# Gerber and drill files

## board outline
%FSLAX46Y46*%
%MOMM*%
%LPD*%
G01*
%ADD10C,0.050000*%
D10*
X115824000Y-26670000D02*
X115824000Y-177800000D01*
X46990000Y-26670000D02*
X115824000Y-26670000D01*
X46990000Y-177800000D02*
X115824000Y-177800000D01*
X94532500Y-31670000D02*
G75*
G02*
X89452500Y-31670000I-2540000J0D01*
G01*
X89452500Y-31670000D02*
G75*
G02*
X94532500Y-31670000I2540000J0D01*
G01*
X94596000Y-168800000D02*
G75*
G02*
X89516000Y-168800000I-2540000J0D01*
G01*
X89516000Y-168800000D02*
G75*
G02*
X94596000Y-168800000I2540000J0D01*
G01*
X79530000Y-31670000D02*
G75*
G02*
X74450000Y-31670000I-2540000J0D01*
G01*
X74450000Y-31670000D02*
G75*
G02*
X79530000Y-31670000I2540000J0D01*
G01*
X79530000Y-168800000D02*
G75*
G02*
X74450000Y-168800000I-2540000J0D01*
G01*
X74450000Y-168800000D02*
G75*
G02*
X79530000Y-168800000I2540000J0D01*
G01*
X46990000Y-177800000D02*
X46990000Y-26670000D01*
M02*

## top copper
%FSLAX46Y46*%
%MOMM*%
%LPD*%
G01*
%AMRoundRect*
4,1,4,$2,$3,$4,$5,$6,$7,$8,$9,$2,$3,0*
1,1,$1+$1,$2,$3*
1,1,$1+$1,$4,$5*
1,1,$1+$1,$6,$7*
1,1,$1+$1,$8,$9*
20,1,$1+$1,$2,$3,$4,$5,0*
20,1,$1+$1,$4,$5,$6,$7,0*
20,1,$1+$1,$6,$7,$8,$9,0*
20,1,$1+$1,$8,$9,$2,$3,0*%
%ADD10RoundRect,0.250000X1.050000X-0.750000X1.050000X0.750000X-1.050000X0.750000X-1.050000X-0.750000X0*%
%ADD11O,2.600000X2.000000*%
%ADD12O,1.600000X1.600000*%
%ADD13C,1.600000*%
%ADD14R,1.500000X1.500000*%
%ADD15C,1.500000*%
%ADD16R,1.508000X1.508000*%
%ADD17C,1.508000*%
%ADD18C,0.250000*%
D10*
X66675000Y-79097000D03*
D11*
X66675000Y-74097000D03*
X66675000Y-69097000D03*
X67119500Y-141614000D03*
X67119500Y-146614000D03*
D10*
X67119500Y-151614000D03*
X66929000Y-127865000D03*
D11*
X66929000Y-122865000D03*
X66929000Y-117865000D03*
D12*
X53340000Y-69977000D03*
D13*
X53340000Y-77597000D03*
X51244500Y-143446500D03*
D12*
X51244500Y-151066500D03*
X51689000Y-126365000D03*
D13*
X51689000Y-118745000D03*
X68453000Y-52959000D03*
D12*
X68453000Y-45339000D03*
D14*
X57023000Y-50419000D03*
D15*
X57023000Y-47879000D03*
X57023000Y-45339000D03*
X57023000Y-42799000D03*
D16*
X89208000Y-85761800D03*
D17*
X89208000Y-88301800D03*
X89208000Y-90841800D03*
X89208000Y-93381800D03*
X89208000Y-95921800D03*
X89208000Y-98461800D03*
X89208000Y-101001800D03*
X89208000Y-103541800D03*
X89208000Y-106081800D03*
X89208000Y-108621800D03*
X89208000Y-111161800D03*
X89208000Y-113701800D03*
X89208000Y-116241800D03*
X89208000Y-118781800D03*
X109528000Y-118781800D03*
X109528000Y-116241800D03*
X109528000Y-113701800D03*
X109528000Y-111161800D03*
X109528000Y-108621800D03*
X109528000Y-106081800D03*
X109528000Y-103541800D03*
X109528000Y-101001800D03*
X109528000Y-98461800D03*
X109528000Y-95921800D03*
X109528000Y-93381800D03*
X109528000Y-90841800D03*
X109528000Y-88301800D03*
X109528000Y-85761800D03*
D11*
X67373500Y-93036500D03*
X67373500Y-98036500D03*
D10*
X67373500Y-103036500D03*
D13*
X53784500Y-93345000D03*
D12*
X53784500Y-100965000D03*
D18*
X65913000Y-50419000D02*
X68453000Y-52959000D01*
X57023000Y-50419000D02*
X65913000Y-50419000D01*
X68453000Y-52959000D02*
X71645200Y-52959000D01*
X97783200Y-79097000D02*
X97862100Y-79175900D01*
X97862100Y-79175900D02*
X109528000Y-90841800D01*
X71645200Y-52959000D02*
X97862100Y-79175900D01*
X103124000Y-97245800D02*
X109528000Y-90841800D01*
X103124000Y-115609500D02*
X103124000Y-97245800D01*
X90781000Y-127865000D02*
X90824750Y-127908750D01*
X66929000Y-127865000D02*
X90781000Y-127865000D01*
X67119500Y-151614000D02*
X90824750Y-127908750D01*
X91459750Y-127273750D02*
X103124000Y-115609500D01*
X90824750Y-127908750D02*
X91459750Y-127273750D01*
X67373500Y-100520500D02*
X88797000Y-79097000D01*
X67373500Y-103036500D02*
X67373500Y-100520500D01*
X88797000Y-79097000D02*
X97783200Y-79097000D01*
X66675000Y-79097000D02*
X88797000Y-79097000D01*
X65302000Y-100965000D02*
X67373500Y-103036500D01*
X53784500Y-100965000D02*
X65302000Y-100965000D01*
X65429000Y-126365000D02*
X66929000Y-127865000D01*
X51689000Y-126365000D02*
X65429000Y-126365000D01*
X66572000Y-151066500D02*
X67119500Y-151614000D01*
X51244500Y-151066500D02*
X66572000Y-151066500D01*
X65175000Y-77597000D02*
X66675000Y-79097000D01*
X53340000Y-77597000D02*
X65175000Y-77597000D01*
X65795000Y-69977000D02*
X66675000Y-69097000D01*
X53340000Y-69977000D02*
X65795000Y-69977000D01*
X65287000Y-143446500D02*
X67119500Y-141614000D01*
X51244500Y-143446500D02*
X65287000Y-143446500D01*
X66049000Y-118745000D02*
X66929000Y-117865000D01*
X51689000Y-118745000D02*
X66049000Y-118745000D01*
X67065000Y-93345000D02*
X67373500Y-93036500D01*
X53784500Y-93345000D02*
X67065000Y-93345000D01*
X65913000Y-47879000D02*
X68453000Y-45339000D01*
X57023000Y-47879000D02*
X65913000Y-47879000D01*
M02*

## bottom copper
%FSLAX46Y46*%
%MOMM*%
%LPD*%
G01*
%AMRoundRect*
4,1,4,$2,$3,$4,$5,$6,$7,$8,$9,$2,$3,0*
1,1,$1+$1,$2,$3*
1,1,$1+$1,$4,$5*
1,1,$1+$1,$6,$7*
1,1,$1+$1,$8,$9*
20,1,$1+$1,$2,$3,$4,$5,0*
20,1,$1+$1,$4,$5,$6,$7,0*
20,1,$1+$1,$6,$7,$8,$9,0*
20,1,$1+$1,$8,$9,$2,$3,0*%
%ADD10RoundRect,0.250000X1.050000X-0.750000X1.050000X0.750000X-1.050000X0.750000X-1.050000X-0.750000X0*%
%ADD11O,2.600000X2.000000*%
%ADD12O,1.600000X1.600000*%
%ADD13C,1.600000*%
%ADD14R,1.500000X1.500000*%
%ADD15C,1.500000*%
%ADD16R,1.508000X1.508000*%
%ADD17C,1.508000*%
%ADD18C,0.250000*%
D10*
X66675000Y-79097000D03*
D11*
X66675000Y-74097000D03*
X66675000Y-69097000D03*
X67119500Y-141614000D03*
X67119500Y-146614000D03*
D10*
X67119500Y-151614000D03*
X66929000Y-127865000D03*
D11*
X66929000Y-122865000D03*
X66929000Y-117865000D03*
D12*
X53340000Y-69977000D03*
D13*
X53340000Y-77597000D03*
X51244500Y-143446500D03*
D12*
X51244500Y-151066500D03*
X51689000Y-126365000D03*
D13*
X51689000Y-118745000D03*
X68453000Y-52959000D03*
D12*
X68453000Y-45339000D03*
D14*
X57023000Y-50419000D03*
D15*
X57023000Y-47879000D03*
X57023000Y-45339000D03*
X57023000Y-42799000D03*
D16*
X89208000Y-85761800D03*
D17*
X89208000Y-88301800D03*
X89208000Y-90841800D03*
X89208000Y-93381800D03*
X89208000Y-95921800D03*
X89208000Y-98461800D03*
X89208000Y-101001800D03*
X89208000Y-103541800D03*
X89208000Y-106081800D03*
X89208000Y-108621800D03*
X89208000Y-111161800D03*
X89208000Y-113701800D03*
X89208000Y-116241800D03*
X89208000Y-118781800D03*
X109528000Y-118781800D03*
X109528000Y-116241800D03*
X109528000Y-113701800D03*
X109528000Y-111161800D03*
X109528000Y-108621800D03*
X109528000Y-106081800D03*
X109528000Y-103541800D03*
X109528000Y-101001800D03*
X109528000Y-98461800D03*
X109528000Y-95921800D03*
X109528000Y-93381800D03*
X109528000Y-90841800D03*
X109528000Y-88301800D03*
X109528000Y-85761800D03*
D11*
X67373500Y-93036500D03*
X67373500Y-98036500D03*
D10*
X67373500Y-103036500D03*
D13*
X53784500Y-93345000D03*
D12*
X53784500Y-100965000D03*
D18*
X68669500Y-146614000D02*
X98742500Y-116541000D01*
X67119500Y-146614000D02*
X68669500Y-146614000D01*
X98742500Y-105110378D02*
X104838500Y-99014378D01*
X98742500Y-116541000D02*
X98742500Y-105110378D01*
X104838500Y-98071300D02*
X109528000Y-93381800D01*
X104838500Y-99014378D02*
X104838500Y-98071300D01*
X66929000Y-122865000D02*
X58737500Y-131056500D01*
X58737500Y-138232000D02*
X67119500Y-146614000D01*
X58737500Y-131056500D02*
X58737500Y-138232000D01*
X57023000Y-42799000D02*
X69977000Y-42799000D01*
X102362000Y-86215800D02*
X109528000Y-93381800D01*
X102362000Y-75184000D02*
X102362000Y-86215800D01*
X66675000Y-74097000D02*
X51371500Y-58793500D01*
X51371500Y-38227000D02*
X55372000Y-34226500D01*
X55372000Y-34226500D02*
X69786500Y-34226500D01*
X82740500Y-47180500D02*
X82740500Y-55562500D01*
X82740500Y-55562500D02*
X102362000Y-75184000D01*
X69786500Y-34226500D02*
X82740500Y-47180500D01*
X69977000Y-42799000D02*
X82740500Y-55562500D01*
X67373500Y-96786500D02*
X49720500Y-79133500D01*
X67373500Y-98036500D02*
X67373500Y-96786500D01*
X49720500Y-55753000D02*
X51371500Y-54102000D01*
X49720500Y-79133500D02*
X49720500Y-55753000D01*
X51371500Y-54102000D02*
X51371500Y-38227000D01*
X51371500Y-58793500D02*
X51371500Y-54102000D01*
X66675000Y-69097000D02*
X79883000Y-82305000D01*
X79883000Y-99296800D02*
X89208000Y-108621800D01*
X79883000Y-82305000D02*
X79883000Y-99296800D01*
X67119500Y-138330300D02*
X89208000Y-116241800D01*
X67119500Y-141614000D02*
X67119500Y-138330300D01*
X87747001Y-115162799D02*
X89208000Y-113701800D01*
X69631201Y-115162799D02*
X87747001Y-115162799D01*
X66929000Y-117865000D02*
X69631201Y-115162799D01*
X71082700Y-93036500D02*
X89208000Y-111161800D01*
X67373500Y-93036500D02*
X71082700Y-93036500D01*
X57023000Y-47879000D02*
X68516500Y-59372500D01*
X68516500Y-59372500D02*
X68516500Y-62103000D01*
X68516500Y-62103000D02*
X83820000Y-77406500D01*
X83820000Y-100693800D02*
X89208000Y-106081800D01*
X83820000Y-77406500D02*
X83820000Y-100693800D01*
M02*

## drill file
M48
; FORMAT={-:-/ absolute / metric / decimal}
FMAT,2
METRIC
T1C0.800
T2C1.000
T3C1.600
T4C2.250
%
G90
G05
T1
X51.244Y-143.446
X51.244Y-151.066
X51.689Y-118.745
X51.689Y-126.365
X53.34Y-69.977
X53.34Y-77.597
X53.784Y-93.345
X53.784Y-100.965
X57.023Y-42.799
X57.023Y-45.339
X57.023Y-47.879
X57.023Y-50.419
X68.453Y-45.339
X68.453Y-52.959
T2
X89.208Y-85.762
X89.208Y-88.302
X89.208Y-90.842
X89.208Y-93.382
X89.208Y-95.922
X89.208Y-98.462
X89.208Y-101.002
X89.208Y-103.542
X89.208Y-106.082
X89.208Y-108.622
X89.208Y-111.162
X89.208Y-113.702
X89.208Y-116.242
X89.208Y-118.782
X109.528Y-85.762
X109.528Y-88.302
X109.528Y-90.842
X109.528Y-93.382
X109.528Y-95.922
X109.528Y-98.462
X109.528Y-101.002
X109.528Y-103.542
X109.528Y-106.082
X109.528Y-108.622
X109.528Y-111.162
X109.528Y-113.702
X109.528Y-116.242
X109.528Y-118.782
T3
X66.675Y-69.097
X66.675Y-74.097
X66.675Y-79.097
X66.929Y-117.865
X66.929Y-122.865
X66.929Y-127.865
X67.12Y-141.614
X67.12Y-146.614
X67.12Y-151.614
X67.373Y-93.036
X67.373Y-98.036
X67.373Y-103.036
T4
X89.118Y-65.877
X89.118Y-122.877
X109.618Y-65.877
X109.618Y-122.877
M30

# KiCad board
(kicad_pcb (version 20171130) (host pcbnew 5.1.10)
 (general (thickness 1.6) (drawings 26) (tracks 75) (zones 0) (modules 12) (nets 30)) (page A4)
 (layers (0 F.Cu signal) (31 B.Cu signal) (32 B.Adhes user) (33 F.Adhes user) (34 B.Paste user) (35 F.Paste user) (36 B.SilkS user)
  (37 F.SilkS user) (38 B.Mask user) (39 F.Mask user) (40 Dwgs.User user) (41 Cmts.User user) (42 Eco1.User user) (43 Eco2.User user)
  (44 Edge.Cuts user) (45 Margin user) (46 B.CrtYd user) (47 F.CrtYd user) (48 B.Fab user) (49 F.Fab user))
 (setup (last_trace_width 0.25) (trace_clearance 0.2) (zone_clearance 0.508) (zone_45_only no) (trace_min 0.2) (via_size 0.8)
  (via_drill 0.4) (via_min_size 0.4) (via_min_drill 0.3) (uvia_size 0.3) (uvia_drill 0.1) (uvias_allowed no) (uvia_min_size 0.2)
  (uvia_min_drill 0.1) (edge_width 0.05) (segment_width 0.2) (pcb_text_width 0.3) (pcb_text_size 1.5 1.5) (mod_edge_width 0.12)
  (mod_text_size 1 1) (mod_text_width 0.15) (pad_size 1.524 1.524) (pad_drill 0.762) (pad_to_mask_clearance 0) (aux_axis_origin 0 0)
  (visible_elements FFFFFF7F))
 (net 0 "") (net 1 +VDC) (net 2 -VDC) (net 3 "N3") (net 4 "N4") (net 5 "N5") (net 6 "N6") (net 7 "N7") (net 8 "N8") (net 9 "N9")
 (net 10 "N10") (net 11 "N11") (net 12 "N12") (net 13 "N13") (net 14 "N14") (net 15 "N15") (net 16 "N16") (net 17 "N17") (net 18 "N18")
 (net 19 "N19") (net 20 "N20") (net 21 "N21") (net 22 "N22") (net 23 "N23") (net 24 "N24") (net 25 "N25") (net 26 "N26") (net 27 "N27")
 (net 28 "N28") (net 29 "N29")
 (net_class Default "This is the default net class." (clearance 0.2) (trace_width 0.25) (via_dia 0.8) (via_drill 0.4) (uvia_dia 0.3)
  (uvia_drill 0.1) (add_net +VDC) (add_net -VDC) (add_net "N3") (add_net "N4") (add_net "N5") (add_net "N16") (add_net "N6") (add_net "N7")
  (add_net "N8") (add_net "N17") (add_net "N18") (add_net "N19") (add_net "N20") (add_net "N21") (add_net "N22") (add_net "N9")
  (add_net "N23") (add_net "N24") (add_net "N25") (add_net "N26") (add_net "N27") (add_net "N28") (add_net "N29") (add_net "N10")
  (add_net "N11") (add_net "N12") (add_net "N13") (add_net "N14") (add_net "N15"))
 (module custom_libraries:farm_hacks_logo (layer F.Cu) (at 102.108 146.304)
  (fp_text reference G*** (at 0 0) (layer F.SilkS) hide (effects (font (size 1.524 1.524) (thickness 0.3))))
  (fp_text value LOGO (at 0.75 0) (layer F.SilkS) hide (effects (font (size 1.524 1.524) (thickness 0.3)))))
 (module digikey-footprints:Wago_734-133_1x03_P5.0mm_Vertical (layer F.Cu) (at 66.675 77.597 90)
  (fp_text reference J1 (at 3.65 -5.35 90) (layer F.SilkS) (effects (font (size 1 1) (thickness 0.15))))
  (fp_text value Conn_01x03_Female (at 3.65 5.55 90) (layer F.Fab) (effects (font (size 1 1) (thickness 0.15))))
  (pad 1 thru_hole roundrect (at -1.5 0 90) (size 2 2.6) (drill 1.6) (layers *.Cu *.Mask) (roundrect_rratio 0.125) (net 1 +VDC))
  (pad 2 thru_hole oval (at 3.5 0 90) (size 2 2.6) (drill 1.6) (layers *.Cu *.Mask) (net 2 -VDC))
  (pad 3 thru_hole oval (at 8.5 0 90) (size 2 2.6) (drill 1.6) (layers *.Cu *.Mask) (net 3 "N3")))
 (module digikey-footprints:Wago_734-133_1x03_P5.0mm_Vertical (layer F.Cu) (at 67.1195 150.114 90)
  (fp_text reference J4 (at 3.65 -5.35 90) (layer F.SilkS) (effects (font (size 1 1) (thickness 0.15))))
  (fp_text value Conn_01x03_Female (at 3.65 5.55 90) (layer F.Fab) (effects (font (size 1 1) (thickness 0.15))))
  (pad 3 thru_hole oval (at 8.5 0 90) (size 2 2.6) (drill 1.6) (layers *.Cu *.Mask) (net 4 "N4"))
  (pad 2 thru_hole oval (at 3.5 0 90) (size 2 2.6) (drill 1.6) (layers *.Cu *.Mask) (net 2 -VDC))
  (pad 1 thru_hole roundrect (at -1.5 0 90) (size 2 2.6) (drill 1.6) (layers *.Cu *.Mask) (roundrect_rratio 0.125) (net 1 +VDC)))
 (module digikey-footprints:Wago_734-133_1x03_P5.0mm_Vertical (layer F.Cu) (at 66.929 126.365 90)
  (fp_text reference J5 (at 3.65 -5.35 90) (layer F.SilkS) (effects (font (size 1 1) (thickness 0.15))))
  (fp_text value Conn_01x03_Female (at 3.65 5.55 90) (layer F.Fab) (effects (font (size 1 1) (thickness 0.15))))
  (pad 1 thru_hole roundrect (at -1.5 0 90) (size 2 2.6) (drill 1.6) (layers *.Cu *.Mask) (roundrect_rratio 0.125) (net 1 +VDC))
  (pad 2 thru_hole oval (at 3.5 0 90) (size 2 2.6) (drill 1.6) (layers *.Cu *.Mask) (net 2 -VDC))
  (pad 3 thru_hole oval (at 8.5 0 90) (size 2 2.6) (drill 1.6) (layers *.Cu *.Mask) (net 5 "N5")))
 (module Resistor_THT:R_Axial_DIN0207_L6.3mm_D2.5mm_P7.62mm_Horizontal (layer F.Cu) (at 53.34 77.597 90)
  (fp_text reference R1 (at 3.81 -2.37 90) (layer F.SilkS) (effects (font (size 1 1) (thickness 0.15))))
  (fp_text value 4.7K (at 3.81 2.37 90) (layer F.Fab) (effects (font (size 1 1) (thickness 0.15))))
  (pad 2 thru_hole oval (at 7.62 0 90) (size 1.6 1.6) (drill 0.8) (layers *.Cu *.Mask) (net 3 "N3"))
  (pad 1 thru_hole circle (at 0 0 90) (size 1.6 1.6) (drill 0.8) (layers *.Cu *.Mask) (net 1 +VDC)))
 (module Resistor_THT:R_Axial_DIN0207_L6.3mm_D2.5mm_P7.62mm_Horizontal (layer F.Cu) (at 51.2445 143.4465 270)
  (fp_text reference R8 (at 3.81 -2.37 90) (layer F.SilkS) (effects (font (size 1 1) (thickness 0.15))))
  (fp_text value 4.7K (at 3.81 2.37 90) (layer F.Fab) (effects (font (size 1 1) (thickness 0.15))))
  (pad 1 thru_hole circle (at 0 0 270) (size 1.6 1.6) (drill 0.8) (layers *.Cu *.Mask) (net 4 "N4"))
  (pad 2 thru_hole oval (at 7.62 0 270) (size 1.6 1.6) (drill 0.8) (layers *.Cu *.Mask) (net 1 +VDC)))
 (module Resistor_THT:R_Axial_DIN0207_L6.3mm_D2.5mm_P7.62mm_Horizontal (layer F.Cu) (at 51.689 118.745 270)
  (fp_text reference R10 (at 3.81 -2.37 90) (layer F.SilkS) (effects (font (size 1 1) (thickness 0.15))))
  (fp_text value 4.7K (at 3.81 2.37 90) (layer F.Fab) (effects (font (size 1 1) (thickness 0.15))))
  (pad 2 thru_hole oval (at 7.62 0 270) (size 1.6 1.6) (drill 0.8) (layers *.Cu *.Mask) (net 1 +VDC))
  (pad 1 thru_hole circle (at 0 0 270) (size 1.6 1.6) (drill 0.8) (layers *.Cu *.Mask) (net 5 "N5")))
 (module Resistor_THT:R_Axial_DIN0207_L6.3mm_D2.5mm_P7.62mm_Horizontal (layer F.Cu) (at 68.453 52.959 90)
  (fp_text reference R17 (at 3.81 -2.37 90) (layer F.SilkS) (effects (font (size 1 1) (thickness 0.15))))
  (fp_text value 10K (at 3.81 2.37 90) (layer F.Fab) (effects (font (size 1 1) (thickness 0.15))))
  (pad 1 thru_hole circle (at 0 0 90) (size 1.6 1.6) (drill 0.8) (layers *.Cu *.Mask) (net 1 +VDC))
  (pad 2 thru_hole oval (at 7.62 0 90) (size 1.6 1.6) (drill 0.8) (layers *.Cu *.Mask) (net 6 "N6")))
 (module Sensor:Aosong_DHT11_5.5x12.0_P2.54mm (layer F.Cu) (at 57.023 50.419 180)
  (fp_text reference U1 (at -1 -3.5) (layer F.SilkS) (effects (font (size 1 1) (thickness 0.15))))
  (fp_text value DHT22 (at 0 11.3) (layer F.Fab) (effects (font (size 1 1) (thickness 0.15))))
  (pad 1 thru_hole rect (at 0 0 180) (size 1.5 1.5) (drill 0.8) (layers *.Cu *.Mask) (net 1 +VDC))
  (pad 2 thru_hole circle (at 0 2.54 180) (size 1.5 1.5) (drill 0.8) (layers *.Cu *.Mask) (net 6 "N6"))
  (pad 3 thru_hole circle (at 0 5.08 180) (size 1.5 1.5) (drill 0.8) (layers *.Cu *.Mask) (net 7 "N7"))
  (pad 4 thru_hole circle (at 0 7.62 180) (size 1.5 1.5) (drill 0.8) (layers *.Cu *.Mask) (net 2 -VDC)))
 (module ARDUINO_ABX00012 (layer F.Cu) (at 86.868 63.627 270)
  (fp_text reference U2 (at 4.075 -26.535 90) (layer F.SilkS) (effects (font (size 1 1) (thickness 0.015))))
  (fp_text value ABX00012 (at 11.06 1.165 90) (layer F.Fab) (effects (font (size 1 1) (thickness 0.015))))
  (pad 1 thru_hole rect (at 22.1348 -2.34 270) (size 1.508 1.508) (drill 1) (layers *.Cu *.Mask) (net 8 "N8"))
  (pad 2 thru_hole circle (at 24.6748 -2.34 270) (size 1.508 1.508) (drill 1) (layers *.Cu *.Mask) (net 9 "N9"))
  (pad 3 thru_hole circle (at 27.2148 -2.34 270) (size 1.508 1.508) (drill 1) (layers *.Cu *.Mask) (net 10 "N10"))
  (pad 4 thru_hole circle (at 29.7548 -2.34 270) (size 1.508 1.508) (drill 1) (layers *.Cu *.Mask) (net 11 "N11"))
  (pad 5 thru_hole circle (at 32.2948 -2.34 270) (size 1.508 1.508) (drill 1) (layers *.Cu *.Mask) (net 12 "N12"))
  (pad 6 thru_hole circle (at 34.8348 -2.34 270) (size 1.508 1.508) (drill 1) (layers *.Cu *.Mask) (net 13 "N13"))
  (pad 7 thru_hole circle (at 37.3748 -2.34 270) (size 1.508 1.508) (drill 1) (layers *.Cu *.Mask) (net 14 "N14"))
  (pad 8 thru_hole circle (at 39.9148 -2.34 270) (size 1.508 1.508) (drill 1) (layers *.Cu *.Mask) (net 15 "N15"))
  (pad 9 thru_hole circle (at 42.4548 -2.34 270) (size 1.508 1.508) (drill 1) (layers *.Cu *.Mask) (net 6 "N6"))
  (pad 10 thru_hole circle (at 44.9948 -2.34 270) (size 1.508 1.508) (drill 1) (layers *.Cu *.Mask) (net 3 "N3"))
  (pad 11 thru_hole circle (at 47.5348 -2.34 270) (size 1.508 1.508) (drill 1) (layers *.Cu *.Mask) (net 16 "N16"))
  (pad 12 thru_hole circle (at 50.0748 -2.34 270) (size 1.508 1.508) (drill 1) (layers *.Cu *.Mask) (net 5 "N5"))
  (pad 13 thru_hole circle (at 52.6148 -2.34 270) (size 1.508 1.508) (drill 1) (layers *.Cu *.Mask) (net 4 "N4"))
  (pad 14 thru_hole circle (at 55.1548 -2.34 270) (size 1.508 1.508) (drill 1) (layers *.Cu *.Mask) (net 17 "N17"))
  (pad 15 thru_hole circle (at 55.1548 -22.66 270) (size 1.508 1.508) (drill 1) (layers *.Cu *.Mask) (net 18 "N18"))
  (pad 16 thru_hole circle (at 52.6148 -22.66 270) (size 1.508 1.508) (drill 1) (layers *.Cu *.Mask) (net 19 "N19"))
  (pad 17 thru_hole circle (at 50.0748 -22.66 270) (size 1.508 1.508) (drill 1) (layers *.Cu *.Mask) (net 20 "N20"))
  (pad 18 thru_hole circle (at 47.5348 -22.66 270) (size 1.508 1.508) (drill 1) (layers *.Cu *.Mask) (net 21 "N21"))
  (pad 19 thru_hole circle (at 44.9948 -22.66 270) (size 1.508 1.508) (drill 1) (layers *.Cu *.Mask) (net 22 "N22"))
  (pad 20 thru_hole circle (at 42.4548 -22.66 270) (size 1.508 1.508) (drill 1) (layers *.Cu *.Mask) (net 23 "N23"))
  (pad 21 thru_hole circle (at 39.9148 -22.66 270) (size 1.508 1.508) (drill 1) (layers *.Cu *.Mask) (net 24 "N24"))
  (pad 22 thru_hole circle (at 37.3748 -22.66 270) (size 1.508 1.508) (drill 1) (layers *.Cu *.Mask) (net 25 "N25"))
  (pad 23 thru_hole circle (at 34.8348 -22.66 270) (size 1.508 1.508) (drill 1) (layers *.Cu *.Mask) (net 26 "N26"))
  (pad 24 thru_hole circle (at 32.2948 -22.66 270) (size 1.508 1.508) (drill 1) (layers *.Cu *.Mask) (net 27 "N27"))
  (pad 25 thru_hole circle (at 29.7548 -22.66 270) (size 1.508 1.508) (drill 1) (layers *.Cu *.Mask) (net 2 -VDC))
  (pad 26 thru_hole circle (at 27.2148 -22.66 270) (size 1.508 1.508) (drill 1) (layers *.Cu *.Mask) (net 1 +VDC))
  (pad 27 thru_hole circle (at 24.6748 -22.66 270) (size 1.508 1.508) (drill 1) (layers *.Cu *.Mask) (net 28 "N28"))
  (pad 28 thru_hole circle (at 22.1348 -22.66 270) (size 1.508 1.508) (drill 1) (layers *.Cu *.Mask) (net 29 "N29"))
  (pad None np_thru_hole circle (at 2.25 -2.25 270) (size 2.25 2.25) (drill 2.25) (layers *.Cu *.Mask))
  (pad None np_thru_hole circle (at 2.25 -22.75 270) (size 2.25 2.25) (drill 2.25) (layers *.Cu *.Mask))
  (pad None np_thru_hole circle (at 59.25 -22.75 270) (size 2.25 2.25) (drill 2.25) (layers *.Cu *.Mask))
  (pad None np_thru_hole circle (at 59.25 -2.25 270) (size 2.25 2.25) (drill 2.25) (layers *.Cu *.Mask)))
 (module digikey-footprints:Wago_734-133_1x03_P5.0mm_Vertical (layer F.Cu) (at 67.3735 101.5365 90)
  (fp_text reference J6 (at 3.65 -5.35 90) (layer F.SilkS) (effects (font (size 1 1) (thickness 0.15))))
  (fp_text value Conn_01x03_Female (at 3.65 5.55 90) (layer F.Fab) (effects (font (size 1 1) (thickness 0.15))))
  (pad 3 thru_hole oval (at 8.5 0 90) (size 2 2.6) (drill 1.6) (layers *.Cu *.Mask) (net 16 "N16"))
  (pad 2 thru_hole oval (at 3.5 0 90) (size 2 2.6) (drill 1.6) (layers *.Cu *.Mask) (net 2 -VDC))
  (pad 1 thru_hole roundrect (at -1.5 0 90) (size 2 2.6) (drill 1.6) (layers *.Cu *.Mask) (roundrect_rratio 0.125) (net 1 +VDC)))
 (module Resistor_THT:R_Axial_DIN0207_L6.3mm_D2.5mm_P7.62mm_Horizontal (layer F.Cu) (at 53.7845 93.345 270)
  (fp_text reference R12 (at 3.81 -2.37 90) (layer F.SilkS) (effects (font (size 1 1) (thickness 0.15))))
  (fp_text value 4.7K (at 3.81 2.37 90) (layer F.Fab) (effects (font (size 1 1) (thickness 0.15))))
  (pad 1 thru_hole circle (at 0 0 270) (size 1.6 1.6) (drill 0.8) (layers *.Cu *.Mask) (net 16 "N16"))
  (pad 2 thru_hole oval (at 7.62 0 270) (size 1.6 1.6) (drill 0.8) (layers *.Cu *.Mask) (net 1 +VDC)))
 (gr_line (start 115.824 26.67) (end 115.824 177.8) (layer Edge.Cuts) (width 0.05))
 (gr_line (start 46.99 26.67) (end 115.824 26.67) (layer Edge.Cuts) (width 0.05))
 (gr_line (start 46.99 177.8) (end 115.824 177.8) (layer Edge.Cuts) (width 0.05))
 (gr_circle (center 91.9925 31.67) (end 91.9925 34.21) (layer Edge.Cuts) (width 0.05))
 (gr_circle (center 92.056 168.8) (end 92.056 166.26) (layer Edge.Cuts) (width 0.05))
 (gr_circle (center 76.99 31.67) (end 76.99 34.21) (layer Edge.Cuts) (width 0.05))
 (gr_circle (center 76.99 168.8) (end 76.99 166.26) (layer Edge.Cuts) (width 0.05))
 (gr_line (start 46.99 177.8) (end 46.99 26.67) (layer Edge.Cuts) (width 0.05))
 (segment (start 65.913 50.419) (end 68.453 52.959) (width 0.25) (layer F.Cu) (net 1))
 (segment (start 57.023 50.419) (end 65.913 50.419) (width 0.25) (layer F.Cu) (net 1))
 (segment (start 68.453 52.959) (end 71.6452 52.959) (width 0.25) (layer F.Cu) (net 1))
 (segment (start 97.7832 79.097) (end 97.8621 79.1759) (width 0.25) (layer F.Cu) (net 1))
 (segment (start 97.8621 79.1759) (end 109.528 90.8418) (width 0.25) (layer F.Cu) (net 1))
 (segment (start 71.6452 52.959) (end 97.8621 79.1759) (width 0.25) (layer F.Cu) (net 1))
 (segment (start 103.124 97.2458) (end 109.528 90.8418) (width 0.25) (layer F.Cu) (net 1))
 (segment (start 103.124 115.6095) (end 103.124 97.2458) (width 0.25) (layer F.Cu) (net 1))
 (segment (start 90.781 127.865) (end 90.82475 127.90875) (width 0.25) (layer F.Cu) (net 1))
 (segment (start 66.929 127.865) (end 90.781 127.865) (width 0.25) (layer F.Cu) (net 1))
 (segment (start 67.1195 151.614) (end 90.82475 127.90875) (width 0.25) (layer F.Cu) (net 1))
 (segment (start 91.45975 127.27375) (end 103.124 115.6095) (width 0.25) (layer F.Cu) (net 1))
 (segment (start 90.82475 127.90875) (end 91.45975 127.27375) (width 0.25) (layer F.Cu) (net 1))
 (segment (start 67.3735 100.5205) (end 88.797 79.097) (width 0.25) (layer F.Cu) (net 1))
 (segment (start 67.3735 103.0365) (end 67.3735 100.5205) (width 0.25) (layer F.Cu) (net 1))
 (segment (start 88.797 79.097) (end 97.7832 79.097) (width 0.25) (layer F.Cu) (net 1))
 (segment (start 66.675 79.097) (end 88.797 79.097) (width 0.25) (layer F.Cu) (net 1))
 (segment (start 65.302 100.965) (end 67.3735 103.0365) (width 0.25) (layer F.Cu) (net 1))
 (segment (start 53.7845 100.965) (end 65.302 100.965) (width 0.25) (layer F.Cu) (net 1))
 (segment (start 65.429 126.365) (end 66.929 127.865) (width 0.25) (layer F.Cu) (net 1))
 (segment (start 51.689 126.365) (end 65.429 126.365) (width 0.25) (layer F.Cu) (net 1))
 (segment (start 66.572 151.0665) (end 67.1195 151.614) (width 0.25) (layer F.Cu) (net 1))
 (segment (start 51.2445 151.0665) (end 66.572 151.0665) (width 0.25) (layer F.Cu) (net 1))
 (segment (start 65.175 77.597) (end 66.675 79.097) (width 0.25) (layer F.Cu) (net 1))
 (segment (start 53.34 77.597) (end 65.175 77.597) (width 0.25) (layer F.Cu) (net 1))
 (segment (start 68.6695 146.614) (end 98.7425 116.541) (width 0.25) (layer B.Cu) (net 2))
 (segment (start 67.1195 146.614) (end 68.6695 146.614) (width 0.25) (layer B.Cu) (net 2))
 (segment (start 98.7425 105.110378) (end 104.8385 99.014378) (width 0.25) (layer B.Cu) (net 2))
 (segment (start 98.7425 116.541) (end 98.7425 105.110378) (width 0.25) (layer B.Cu) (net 2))
 (segment (start 104.8385 98.0713) (end 109.528 93.3818) (width 0.25) (layer B.Cu) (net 2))
 (segment (start 104.8385 99.014378) (end 104.8385 98.0713) (width 0.25) (layer B.Cu) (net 2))
 (segment (start 66.929 122.865) (end 58.7375 131.0565) (width 0.25) (layer B.Cu) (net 2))
 (segment (start 58.7375 138.232) (end 67.1195 146.614) (width 0.25) (layer B.Cu) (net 2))
 (segment (start 58.7375 131.0565) (end 58.7375 138.232) (width 0.25) (layer B.Cu) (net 2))
 (segment (start 57.023 42.799) (end 69.977 42.799) (width 0.25) (layer B.Cu) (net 2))
 (segment (start 102.362 86.2158) (end 109.528 93.3818) (width 0.25) (layer B.Cu) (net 2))
 (segment (start 102.362 75.184) (end 102.362 86.2158) (width 0.25) (layer B.Cu) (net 2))
 (segment (start 66.675 74.097) (end 51.3715 58.7935) (width 0.25) (layer B.Cu) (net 2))
 (segment (start 51.3715 38.227) (end 55.372 34.2265) (width 0.25) (layer B.Cu) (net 2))
 (segment (start 55.372 34.2265) (end 69.7865 34.2265) (width 0.25) (layer B.Cu) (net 2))
 (segment (start 82.7405 47.1805) (end 82.7405 55.5625) (width 0.25) (layer B.Cu) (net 2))
 (segment (start 82.7405 55.5625) (end 102.362 75.184) (width 0.25) (layer B.Cu) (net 2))
 (segment (start 69.7865 34.2265) (end 82.7405 47.1805) (width 0.25) (layer B.Cu) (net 2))
 (segment (start 69.977 42.799) (end 82.7405 55.5625) (width 0.25) (layer B.Cu) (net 2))
 (segment (start 67.3735 96.7865) (end 49.7205 79.1335) (width 0.25) (layer B.Cu) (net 2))
 (segment (start 67.3735 98.0365) (end 67.3735 96.7865) (width 0.25) (layer B.Cu) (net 2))
 (segment (start 49.7205 55.753) (end 51.3715 54.102) (width 0.25) (layer B.Cu) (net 2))
 (segment (start 49.7205 79.1335) (end 49.7205 55.753) (width 0.25) (layer B.Cu) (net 2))
 (segment (start 51.3715 54.102) (end 51.3715 38.227) (width 0.25) (layer B.Cu) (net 2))
 (segment (start 51.3715 58.7935) (end 51.3715 54.102) (width 0.25) (layer B.Cu) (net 2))
 (segment (start 66.675 69.097) (end 79.883 82.305) (width 0.25) (layer B.Cu) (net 3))
 (segment (start 79.883 99.2968) (end 89.208 108.6218) (width 0.25) (layer B.Cu) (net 3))
 (segment (start 79.883 82.305) (end 79.883 99.2968) (width 0.25) (layer B.Cu) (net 3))
 (segment (start 65.795 69.977) (end 66.675 69.097) (width 0.25) (layer F.Cu) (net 3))
 (segment (start 53.34 69.977) (end 65.795 69.977) (width 0.25) (layer F.Cu) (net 3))
 (segment (start 67.1195 138.3303) (end 89.208 116.2418) (width 0.25) (layer B.Cu) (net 4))
 (segment (start 67.1195 141.614) (end 67.1195 138.3303) (width 0.25) (layer B.Cu) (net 4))
 (segment (start 65.287 143.4465) (end 67.1195 141.614) (width 0.25) (layer F.Cu) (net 4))
 (segment (start 51.2445 143.4465) (end 65.287 143.4465) (width 0.25) (layer F.Cu) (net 4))
 (segment (start 87.747001 115.162799) (end 89.208 113.7018) (width 0.25) (layer B.Cu) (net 5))
 (segment (start 69.631201 115.162799) (end 87.747001 115.162799) (width 0.25) (layer B.Cu) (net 5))
 (segment (start 66.929 117.865) (end 69.631201 115.162799) (width 0.25) (layer B.Cu) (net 5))
 (segment (start 66.049 118.745) (end 66.929 117.865) (width 0.25) (layer F.Cu) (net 5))
 (segment (start 51.689 118.745) (end 66.049 118.745) (width 0.25) (layer F.Cu) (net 5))
 (segment (start 71.0827 93.0365) (end 89.208 111.1618) (width 0.25) (layer B.Cu) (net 16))
 (segment (start 67.3735 93.0365) (end 71.0827 93.0365) (width 0.25) (layer B.Cu) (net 16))
 (segment (start 67.065 93.345) (end 67.3735 93.0365) (width 0.25) (layer F.Cu) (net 16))
 (segment (start 53.7845 93.345) (end 67.065 93.345) (width 0.25) (layer F.Cu) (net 16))
 (segment (start 57.023 47.879) (end 68.5165 59.3725) (width 0.25) (layer B.Cu) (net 6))
 (segment (start 68.5165 59.3725) (end 68.5165 62.103) (width 0.25) (layer B.Cu) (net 6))
 (segment (start 68.5165 62.103) (end 83.82 77.4065) (width 0.25) (layer B.Cu) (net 6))
 (segment (start 83.82 100.6938) (end 89.208 106.0818) (width 0.25) (layer B.Cu) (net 6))
 (segment (start 83.82 77.4065) (end 83.82 100.6938) (width 0.25) (layer B.Cu) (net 6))
 (segment (start 65.913 47.879) (end 68.453 45.339) (width 0.25) (layer F.Cu) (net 6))
 (segment (start 57.023 47.879) (end 65.913 47.879) (width 0.25) (layer F.Cu) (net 6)))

